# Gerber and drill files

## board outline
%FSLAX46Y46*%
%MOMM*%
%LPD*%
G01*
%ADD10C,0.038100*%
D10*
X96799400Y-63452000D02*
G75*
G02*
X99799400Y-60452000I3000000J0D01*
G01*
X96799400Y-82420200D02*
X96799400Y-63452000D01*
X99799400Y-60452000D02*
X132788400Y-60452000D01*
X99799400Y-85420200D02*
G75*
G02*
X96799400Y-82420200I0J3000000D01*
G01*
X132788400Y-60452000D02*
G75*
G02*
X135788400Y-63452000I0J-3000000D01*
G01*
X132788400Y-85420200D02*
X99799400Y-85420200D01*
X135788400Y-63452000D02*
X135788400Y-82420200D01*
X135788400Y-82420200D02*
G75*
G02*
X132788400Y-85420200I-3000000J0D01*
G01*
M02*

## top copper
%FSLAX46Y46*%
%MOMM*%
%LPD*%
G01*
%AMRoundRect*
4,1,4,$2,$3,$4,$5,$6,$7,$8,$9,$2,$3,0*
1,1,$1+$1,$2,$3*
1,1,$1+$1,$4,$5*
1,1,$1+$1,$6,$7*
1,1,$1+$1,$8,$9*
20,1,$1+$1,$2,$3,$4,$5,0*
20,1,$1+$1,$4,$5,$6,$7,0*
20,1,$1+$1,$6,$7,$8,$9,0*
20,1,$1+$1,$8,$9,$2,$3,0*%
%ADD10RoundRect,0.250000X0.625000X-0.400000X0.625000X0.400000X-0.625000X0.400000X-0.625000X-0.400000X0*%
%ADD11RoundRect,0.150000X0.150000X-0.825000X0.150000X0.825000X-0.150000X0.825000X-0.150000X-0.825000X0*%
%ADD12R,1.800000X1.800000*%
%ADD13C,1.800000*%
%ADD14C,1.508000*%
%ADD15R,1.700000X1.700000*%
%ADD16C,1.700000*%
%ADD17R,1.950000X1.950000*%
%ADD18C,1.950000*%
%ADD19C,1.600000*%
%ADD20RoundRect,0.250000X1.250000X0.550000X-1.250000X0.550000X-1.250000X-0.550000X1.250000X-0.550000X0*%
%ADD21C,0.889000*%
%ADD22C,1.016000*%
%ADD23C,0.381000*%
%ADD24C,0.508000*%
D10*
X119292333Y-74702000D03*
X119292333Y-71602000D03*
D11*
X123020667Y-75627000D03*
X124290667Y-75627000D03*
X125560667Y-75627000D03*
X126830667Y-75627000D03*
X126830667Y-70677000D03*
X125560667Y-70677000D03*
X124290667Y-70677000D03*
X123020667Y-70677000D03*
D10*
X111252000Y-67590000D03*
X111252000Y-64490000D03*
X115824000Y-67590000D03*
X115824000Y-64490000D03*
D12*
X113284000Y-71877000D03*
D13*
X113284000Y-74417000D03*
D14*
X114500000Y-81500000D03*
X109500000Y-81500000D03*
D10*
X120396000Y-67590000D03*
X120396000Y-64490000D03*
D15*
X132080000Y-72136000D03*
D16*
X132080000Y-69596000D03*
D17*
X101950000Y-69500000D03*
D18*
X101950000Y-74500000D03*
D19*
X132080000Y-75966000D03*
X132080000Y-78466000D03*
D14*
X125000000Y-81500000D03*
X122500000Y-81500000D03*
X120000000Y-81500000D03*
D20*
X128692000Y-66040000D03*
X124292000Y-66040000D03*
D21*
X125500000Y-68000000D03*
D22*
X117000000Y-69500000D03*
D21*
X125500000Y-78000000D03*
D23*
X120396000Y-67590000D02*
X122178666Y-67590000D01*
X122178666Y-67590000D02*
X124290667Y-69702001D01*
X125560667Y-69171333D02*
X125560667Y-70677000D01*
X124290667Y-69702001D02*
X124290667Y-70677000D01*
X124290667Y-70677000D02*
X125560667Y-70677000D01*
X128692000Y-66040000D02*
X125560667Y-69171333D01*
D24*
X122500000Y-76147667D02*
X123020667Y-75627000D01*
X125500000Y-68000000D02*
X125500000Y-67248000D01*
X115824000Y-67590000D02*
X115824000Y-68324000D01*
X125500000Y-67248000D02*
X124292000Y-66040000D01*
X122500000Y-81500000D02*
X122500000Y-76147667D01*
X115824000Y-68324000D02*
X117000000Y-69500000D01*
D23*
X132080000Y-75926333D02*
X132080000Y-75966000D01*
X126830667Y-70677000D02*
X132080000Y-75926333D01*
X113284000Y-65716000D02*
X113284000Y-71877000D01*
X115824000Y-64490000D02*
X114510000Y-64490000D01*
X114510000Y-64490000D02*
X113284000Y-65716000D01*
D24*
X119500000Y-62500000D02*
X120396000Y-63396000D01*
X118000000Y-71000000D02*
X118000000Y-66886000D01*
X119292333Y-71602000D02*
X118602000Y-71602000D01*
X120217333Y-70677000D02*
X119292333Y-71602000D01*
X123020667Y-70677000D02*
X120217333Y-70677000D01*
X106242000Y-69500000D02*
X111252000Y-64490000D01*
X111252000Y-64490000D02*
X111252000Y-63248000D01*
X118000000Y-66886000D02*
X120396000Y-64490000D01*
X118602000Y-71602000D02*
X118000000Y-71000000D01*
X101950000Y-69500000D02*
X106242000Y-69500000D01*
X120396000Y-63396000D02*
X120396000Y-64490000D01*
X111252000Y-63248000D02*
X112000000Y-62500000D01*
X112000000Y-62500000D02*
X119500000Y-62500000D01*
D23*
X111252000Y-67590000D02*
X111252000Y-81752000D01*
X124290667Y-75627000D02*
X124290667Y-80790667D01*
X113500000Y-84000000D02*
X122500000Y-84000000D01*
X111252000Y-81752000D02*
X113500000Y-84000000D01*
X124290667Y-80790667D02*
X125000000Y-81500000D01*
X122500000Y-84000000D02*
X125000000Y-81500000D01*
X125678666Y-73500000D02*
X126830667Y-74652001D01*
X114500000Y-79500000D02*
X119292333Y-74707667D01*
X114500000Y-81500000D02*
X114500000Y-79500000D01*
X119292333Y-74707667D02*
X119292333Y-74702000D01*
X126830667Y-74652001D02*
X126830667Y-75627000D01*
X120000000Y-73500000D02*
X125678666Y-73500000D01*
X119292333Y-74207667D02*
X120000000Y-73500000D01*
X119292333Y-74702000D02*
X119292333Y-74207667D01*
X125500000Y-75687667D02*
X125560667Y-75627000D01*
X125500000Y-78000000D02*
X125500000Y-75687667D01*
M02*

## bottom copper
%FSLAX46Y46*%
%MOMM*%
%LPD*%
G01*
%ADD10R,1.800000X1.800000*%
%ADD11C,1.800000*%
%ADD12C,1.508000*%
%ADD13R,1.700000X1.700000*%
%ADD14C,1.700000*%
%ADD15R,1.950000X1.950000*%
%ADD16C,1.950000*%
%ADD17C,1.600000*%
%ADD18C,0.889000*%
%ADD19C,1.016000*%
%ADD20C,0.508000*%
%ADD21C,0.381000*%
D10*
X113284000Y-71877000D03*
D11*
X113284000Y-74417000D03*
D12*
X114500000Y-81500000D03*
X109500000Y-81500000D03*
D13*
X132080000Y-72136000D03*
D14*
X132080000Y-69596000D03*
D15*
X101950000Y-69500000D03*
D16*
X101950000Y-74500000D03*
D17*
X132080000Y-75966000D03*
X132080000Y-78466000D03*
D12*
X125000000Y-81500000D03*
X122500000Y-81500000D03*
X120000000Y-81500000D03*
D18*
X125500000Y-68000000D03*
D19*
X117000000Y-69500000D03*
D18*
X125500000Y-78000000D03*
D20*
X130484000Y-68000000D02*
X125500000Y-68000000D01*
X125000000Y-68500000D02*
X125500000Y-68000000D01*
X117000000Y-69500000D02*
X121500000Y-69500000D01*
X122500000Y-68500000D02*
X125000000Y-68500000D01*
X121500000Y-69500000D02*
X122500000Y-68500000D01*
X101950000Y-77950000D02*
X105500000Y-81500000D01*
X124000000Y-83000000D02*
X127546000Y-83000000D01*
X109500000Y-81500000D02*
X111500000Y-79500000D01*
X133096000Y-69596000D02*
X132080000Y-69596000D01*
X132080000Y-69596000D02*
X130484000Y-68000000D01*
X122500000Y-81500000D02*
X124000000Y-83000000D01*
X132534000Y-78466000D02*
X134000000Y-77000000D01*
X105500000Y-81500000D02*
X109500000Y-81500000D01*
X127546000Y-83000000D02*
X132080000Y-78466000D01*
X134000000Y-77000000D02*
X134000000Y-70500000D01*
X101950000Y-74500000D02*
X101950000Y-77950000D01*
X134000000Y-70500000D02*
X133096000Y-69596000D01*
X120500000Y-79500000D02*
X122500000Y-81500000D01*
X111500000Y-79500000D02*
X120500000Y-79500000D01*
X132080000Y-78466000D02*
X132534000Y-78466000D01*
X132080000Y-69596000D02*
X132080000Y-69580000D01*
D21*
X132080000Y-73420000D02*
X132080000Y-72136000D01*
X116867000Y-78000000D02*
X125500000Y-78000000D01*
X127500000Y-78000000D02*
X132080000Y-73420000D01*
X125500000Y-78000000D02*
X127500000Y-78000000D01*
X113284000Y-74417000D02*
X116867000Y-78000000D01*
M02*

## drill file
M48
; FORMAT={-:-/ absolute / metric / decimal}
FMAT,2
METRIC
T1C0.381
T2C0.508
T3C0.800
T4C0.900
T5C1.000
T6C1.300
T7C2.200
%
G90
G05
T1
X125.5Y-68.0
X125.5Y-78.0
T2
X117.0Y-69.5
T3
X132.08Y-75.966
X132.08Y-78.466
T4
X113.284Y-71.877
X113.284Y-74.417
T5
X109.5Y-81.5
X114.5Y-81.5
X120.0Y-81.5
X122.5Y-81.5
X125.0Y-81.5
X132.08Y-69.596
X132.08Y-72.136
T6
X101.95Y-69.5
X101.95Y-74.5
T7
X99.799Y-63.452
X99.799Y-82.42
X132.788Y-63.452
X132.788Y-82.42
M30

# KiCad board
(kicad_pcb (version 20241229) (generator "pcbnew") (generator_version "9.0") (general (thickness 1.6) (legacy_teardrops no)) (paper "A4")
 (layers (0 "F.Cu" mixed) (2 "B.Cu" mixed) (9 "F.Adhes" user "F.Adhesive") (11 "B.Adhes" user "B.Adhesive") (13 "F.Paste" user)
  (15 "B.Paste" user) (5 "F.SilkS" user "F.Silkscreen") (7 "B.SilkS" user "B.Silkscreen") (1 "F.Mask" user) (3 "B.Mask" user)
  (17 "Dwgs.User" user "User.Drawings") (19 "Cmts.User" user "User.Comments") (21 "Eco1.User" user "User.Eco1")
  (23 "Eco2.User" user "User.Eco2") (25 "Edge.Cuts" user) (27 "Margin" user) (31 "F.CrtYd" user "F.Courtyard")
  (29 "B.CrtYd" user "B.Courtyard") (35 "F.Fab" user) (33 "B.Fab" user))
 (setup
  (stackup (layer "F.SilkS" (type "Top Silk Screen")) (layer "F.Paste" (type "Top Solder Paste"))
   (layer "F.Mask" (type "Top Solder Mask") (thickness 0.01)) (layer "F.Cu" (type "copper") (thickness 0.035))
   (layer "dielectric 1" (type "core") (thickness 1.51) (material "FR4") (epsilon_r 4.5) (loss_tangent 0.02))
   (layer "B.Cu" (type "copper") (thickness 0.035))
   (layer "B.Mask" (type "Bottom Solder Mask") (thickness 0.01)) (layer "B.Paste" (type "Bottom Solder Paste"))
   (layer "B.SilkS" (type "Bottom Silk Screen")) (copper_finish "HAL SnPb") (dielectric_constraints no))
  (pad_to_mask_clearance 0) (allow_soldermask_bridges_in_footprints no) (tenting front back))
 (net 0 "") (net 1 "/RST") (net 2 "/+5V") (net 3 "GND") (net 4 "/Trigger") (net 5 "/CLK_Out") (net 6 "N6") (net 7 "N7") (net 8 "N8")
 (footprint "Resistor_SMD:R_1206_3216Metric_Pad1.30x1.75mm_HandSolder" (layer "F.Cu") (at 119.292333 73.152 90)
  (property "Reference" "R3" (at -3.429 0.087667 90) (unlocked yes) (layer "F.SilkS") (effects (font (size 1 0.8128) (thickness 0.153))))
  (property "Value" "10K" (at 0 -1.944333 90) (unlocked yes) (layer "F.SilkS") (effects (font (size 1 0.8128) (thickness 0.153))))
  (pad "1" smd roundrect (at -1.55 0 90) (size 1.3 1.75) (layers "F.Cu" "F.Mask" "F.Paste") (roundrect_rratio 0.192308) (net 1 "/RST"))
  (pad "2" smd roundrect (at 1.55 0 90) (size 1.3 1.75) (layers "F.Cu" "F.Mask" "F.Paste") (roundrect_rratio 0.192308) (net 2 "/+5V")))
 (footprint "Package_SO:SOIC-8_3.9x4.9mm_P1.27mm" (layer "F.Cu") (at 124.925667 73.152 90)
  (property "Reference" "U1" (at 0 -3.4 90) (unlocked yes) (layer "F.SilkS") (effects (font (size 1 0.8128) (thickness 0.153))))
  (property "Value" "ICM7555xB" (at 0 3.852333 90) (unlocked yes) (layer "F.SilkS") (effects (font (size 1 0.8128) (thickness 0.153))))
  (pad "1" smd roundrect (at -2.475 -1.905 90) (size 1.95 0.6) (layers "F.Cu" "F.Mask" "F.Paste") (roundrect_rratio 0.25) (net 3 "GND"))
  (pad "2" smd roundrect (at -2.475 -0.635 90) (size 1.95 0.6) (layers "F.Cu" "F.Mask" "F.Paste") (roundrect_rratio 0.25) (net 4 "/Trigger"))
  (pad "3" smd roundrect (at -2.475 0.635 90) (size 1.95 0.6) (layers "F.Cu" "F.Mask" "F.Paste") (roundrect_rratio 0.25) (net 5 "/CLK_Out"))
  (pad "4" smd roundrect (at -2.475 1.905 90) (size 1.95 0.6) (layers "F.Cu" "F.Mask" "F.Paste") (roundrect_rratio 0.25) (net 1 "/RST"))
  (pad "5" smd roundrect (at 2.475 1.905 90) (size 1.95 0.6) (layers "F.Cu" "F.Mask" "F.Paste") (roundrect_rratio 0.25) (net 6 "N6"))
  (pad "6" smd roundrect (at 2.475 0.635 90) (size 1.95 0.6) (layers "F.Cu" "F.Mask" "F.Paste") (roundrect_rratio 0.25) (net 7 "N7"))
  (pad "7" smd roundrect (at 2.475 -0.635 90) (size 1.95 0.6) (layers "F.Cu" "F.Mask" "F.Paste") (roundrect_rratio 0.25) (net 7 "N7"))
  (pad "8" smd roundrect (at 2.475 -1.905 90) (size 1.95 0.6) (layers "F.Cu" "F.Mask" "F.Paste") (roundrect_rratio 0.25) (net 2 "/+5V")))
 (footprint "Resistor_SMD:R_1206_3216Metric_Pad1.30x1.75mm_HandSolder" (layer "F.Cu") (at 111.252 66.04 90)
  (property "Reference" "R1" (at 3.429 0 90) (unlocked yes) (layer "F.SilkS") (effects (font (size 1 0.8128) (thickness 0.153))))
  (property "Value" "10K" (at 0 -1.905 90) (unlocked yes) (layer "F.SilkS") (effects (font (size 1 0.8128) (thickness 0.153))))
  (pad "1" smd roundrect (at -1.55 0 90) (size 1.3 1.75) (layers "F.Cu" "F.Mask" "F.Paste") (roundrect_rratio 0.192308) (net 4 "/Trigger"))
  (pad "2" smd roundrect (at 1.55 0 90) (size 1.3 1.75) (layers "F.Cu" "F.Mask" "F.Paste") (roundrect_rratio 0.192308) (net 2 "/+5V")))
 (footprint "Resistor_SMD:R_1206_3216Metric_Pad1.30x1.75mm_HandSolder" (layer "F.Cu") (at 115.824 66.04 90)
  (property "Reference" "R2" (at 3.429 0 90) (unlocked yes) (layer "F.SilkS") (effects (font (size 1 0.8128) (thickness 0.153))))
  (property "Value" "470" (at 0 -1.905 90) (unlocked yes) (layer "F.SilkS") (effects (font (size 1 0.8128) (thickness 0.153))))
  (pad "1" smd roundrect (at -1.55 0 90) (size 1.3 1.75) (layers "F.Cu" "F.Mask" "F.Paste") (roundrect_rratio 0.192308) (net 3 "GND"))
  (pad "2" smd roundrect (at 1.55 0 90) (size 1.3 1.75) (layers "F.Cu" "F.Mask" "F.Paste") (roundrect_rratio 0.192308) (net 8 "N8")))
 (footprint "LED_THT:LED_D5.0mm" (layer "F.Cu") (at 113.284 71.877 -90)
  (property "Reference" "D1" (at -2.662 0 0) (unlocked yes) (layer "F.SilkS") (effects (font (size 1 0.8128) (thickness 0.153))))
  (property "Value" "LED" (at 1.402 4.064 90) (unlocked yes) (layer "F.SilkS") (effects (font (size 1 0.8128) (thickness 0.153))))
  (pad "1" thru_hole rect (at 0 0 270) (size 1.8 1.8) (drill 0.9) (layers "*.Cu" "*.Mask") (remove_unused_layers no) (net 8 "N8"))
  (pad "2" thru_hole circle (at 2.54 0 270) (size 1.8 1.8) (drill 0.9) (layers "*.Cu" "*.Mask") (remove_unused_layers no) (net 5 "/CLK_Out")))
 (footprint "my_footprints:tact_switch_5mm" (layer "F.Cu") (at 112 81.5 180)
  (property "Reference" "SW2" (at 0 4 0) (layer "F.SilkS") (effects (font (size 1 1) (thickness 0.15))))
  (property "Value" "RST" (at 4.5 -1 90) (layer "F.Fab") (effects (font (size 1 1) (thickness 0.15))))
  (pad "1" thru_hole circle (at -2.5 0 180) (size 1.508 1.508) (drill 1) (layers "*.Cu" "*.Mask") (remove_unused_layers no) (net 1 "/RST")
   (solder_mask_margin 0.102))
  (pad "2" thru_hole circle (at 2.5 0 180) (size 1.508 1.508) (drill 1) (layers "*.Cu" "*.Mask") (remove_unused_layers no) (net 3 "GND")
   (solder_mask_margin 0.102)))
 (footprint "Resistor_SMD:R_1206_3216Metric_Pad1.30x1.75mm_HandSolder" (layer "F.Cu") (at 120.396 66.04 90)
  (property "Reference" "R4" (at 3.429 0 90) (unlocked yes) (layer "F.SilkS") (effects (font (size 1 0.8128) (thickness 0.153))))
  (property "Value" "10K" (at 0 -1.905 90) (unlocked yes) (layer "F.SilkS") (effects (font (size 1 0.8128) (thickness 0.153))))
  (pad "1" smd roundrect (at -1.55 0 90) (size 1.3 1.75) (layers "F.Cu" "F.Mask" "F.Paste") (roundrect_rratio 0.192308) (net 7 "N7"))
  (pad "2" smd roundrect (at 1.55 0 90) (size 1.3 1.75) (layers "F.Cu" "F.Mask" "F.Paste") (roundrect_rratio 0.192308) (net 2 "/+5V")))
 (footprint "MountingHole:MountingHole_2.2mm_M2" (layer "F.Cu") (at 99.7994 63.452)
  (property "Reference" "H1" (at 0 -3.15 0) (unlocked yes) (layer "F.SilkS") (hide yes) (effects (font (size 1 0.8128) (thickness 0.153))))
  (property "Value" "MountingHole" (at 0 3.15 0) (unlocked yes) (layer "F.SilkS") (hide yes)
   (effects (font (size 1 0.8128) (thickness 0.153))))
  (pad "" np_thru_hole circle (at 0 0) (size 2.2 2.2) (drill 2.2) (layers "*.Cu" "*.Mask")))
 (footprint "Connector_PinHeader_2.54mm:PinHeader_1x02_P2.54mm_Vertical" (layer "F.Cu") (at 132.08 72.136 180)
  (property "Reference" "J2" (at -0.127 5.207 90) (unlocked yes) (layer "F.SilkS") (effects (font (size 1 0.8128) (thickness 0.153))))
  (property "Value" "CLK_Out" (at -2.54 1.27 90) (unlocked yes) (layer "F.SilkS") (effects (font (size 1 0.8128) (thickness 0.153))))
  (pad "1" thru_hole rect (at 0 0 180) (size 1.7 1.7) (drill 1) (layers "*.Cu" "*.Mask") (remove_unused_layers no) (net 5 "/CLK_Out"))
  (pad "2" thru_hole circle (at 0 2.54 180) (size 1.7 1.7) (drill 1) (layers "*.Cu" "*.Mask") (remove_unused_layers no) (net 3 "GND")))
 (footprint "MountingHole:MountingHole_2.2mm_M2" (layer "F.Cu") (at 132.7884 82.4202)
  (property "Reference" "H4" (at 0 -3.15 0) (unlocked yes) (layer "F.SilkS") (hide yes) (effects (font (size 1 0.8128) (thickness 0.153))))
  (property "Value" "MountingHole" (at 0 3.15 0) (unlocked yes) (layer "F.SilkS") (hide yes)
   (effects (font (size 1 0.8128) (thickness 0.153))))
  (pad "" np_thru_hole circle (at 0 0) (size 2.2 2.2) (drill 2.2) (layers "*.Cu" "*.Mask")))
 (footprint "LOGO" (layer "F.Cu") (at 105.5 63.5)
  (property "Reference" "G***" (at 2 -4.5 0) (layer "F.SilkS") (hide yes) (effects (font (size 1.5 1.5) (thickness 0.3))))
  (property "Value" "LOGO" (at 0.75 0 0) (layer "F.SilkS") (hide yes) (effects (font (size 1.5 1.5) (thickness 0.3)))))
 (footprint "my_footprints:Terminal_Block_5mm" (layer "F.Cu") (at 101.95 72 -90)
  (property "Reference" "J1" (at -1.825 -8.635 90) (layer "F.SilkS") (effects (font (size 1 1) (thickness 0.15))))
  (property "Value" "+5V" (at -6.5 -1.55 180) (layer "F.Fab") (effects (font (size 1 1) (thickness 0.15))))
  (pad "1" thru_hole rect (at -2.5 0 270) (size 1.95 1.95) (drill 1.3) (layers "*.Cu" "*.Mask") (remove_unused_layers no) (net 2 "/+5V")
   (solder_mask_margin 0.102))
  (pad "2" thru_hole circle (at 2.5 0 270) (size 1.95 1.95) (drill 1.3) (layers "*.Cu" "*.Mask") (remove_unused_layers no) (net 3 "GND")
   (solder_mask_margin 0.102)))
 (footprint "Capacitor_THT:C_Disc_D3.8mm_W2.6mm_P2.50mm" (layer "F.Cu") (at 132.08 75.966 -90)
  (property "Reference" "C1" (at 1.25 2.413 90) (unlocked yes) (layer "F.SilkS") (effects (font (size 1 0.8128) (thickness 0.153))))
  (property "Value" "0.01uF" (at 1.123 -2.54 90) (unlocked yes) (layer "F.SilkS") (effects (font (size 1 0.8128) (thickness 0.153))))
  (pad "1" thru_hole circle (at 0 0 270) (size 1.6 1.6) (drill 0.8) (layers "*.Cu" "*.Mask") (remove_unused_layers no) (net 6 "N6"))
  (pad "2" thru_hole circle (at 2.5 0 270) (size 1.6 1.6) (drill 0.8) (layers "*.Cu" "*.Mask") (remove_unused_layers no) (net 3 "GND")))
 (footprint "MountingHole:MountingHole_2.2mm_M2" (layer "F.Cu") (at 132.7884 63.452)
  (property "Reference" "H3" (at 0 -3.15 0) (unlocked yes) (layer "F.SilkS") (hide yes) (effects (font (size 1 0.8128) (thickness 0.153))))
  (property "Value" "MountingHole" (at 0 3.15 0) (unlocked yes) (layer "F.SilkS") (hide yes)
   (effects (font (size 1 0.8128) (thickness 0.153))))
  (pad "" np_thru_hole circle (at 0 0) (size 2.2 2.2) (drill 2.2) (layers "*.Cu" "*.Mask")))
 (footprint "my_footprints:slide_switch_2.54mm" (layer "F.Cu") (at 122.5 81.5 180)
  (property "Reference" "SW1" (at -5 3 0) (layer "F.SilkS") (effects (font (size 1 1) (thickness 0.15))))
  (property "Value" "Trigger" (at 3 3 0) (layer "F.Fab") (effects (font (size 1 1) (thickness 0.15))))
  (pad "1" thru_hole circle (at -2.5 0 180) (size 1.508 1.508) (drill 1) (layers "*.Cu" "*.Mask") (remove_unused_layers no)
   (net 4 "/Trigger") (solder_mask_margin 0.102))
  (pad "2" thru_hole circle (at 0 0 180) (size 1.508 1.508) (drill 1) (layers "*.Cu" "*.Mask") (remove_unused_layers no) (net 3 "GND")
   (solder_mask_margin 0.102))
  (pad "3" thru_hole circle (at 2.5 0 180) (size 1.508 1.508) (drill 1) (layers "*.Cu" "*.Mask") (remove_unused_layers no)
   (solder_mask_margin 0.102)))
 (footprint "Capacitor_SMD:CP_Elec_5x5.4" (layer "F.Cu") (at 126.492 66.04 180)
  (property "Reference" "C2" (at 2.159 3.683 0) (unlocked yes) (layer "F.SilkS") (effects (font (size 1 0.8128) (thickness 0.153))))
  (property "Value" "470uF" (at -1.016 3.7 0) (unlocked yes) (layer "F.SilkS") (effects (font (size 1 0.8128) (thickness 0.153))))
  (pad "1" smd roundrect (at -2.2 0 180) (size 3 1.6) (layers "F.Cu" "F.Mask" "F.Paste") (roundrect_rratio 0.15625) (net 7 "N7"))
  (pad "2" smd roundrect (at 2.2 0 180) (size 3 1.6) (layers "F.Cu" "F.Mask" "F.Paste") (roundrect_rratio 0.15625) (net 3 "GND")))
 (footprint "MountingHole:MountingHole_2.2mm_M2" (layer "F.Cu") (at 99.7994 82.4202)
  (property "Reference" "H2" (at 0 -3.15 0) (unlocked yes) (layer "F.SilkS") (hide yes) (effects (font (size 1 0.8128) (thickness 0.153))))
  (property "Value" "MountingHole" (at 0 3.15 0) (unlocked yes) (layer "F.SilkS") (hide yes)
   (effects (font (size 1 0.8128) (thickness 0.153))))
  (pad "" np_thru_hole circle (at 0 0) (size 2.2 2.2) (drill 2.2) (layers "*.Cu" "*.Mask")))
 (gr_arc (start 96.7994 63.452) (mid 97.67808 61.33068) (end 99.7994 60.452) (stroke (width 0.0381) (type default)) (layer "Edge.Cuts"))
 (gr_line (start 96.7994 82.4202) (end 96.7994 63.452) (stroke (width 0.0381) (type default)) (layer "Edge.Cuts"))
 (gr_line (start 99.7994 60.452) (end 132.7884 60.452) (stroke (width 0.0381) (type default)) (layer "Edge.Cuts"))
 (gr_arc (start 99.7994 85.4202) (mid 97.67808 84.54152) (end 96.7994 82.4202) (stroke (width 0.0381) (type default)) (layer "Edge.Cuts"))
 (gr_arc (start 132.7884 60.452) (mid 134.90972 61.33068) (end 135.7884 63.452) (stroke (width 0.0381) (type default)) (layer "Edge.Cuts"))
 (gr_line (start 132.7884 85.4202) (end 99.7994 85.4202) (stroke (width 0.0381) (type default)) (layer "Edge.Cuts"))
 (gr_line (start 135.7884 63.452) (end 135.7884 82.4202) (stroke (width 0.0381) (type default)) (layer "Edge.Cuts"))
 (gr_arc (start 135.7884 82.4202) (mid 134.90972 84.54152) (end 132.7884 85.4202) (stroke (width 0.0381) (type default)) (layer "Edge.Cuts"))
 (segment (start 120.396 67.59) (end 122.178666 67.59) (width 0.381) (layer "F.Cu") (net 7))
 (segment (start 122.178666 67.59) (end 124.290667 69.702001) (width 0.381) (layer "F.Cu") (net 7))
 (segment (start 125.560667 69.171333) (end 125.560667 70.677) (width 0.381) (layer "F.Cu") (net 7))
 (segment (start 124.290667 69.702001) (end 124.290667 70.677) (width 0.381) (layer "F.Cu") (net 7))
 (segment (start 124.290667 70.677) (end 125.560667 70.677) (width 0.381) (layer "F.Cu") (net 7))
 (segment (start 128.692 66.04) (end 125.560667 69.171333) (width 0.381) (layer "F.Cu") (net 7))
 (segment (start 122.5 76.147667) (end 123.020667 75.627) (width 0.508) (layer "F.Cu") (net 3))
 (segment (start 125.5 68) (end 125.5 67.248) (width 0.508) (layer "F.Cu") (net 3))
 (segment (start 115.824 67.59) (end 115.824 68.324) (width 0.508) (layer "F.Cu") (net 3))
 (segment (start 125.5 67.248) (end 124.292 66.04) (width 0.508) (layer "F.Cu") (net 3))
 (segment (start 122.5 81.5) (end 122.5 76.147667) (width 0.508) (layer "F.Cu") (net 3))
 (segment (start 115.824 68.324) (end 117 69.5) (width 0.508) (layer "F.Cu") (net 3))
 (via (at 125.5 68) (size 0.889) (drill 0.381) (layers "F.Cu" "B.Cu") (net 3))
 (via (at 117 69.5) (size 1.016) (drill 0.508) (layers "F.Cu" "B.Cu") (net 3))
 (segment (start 130.484 68) (end 125.5 68) (width 0.508) (layer "B.Cu") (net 3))
 (segment (start 125 68.5) (end 125.5 68) (width 0.508) (layer "B.Cu") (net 3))
 (segment (start 117 69.5) (end 121.5 69.5) (width 0.508) (layer "B.Cu") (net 3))
 (segment (start 122.5 68.5) (end 125 68.5) (width 0.508) (layer "B.Cu") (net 3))
 (segment (start 121.5 69.5) (end 122.5 68.5) (width 0.508) (layer "B.Cu") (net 3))
 (segment (start 101.95 77.95) (end 105.5 81.5) (width 0.508) (layer "B.Cu") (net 3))
 (segment (start 124 83) (end 127.546 83) (width 0.508) (layer "B.Cu") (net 3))
 (segment (start 109.5 81.5) (end 111.5 79.5) (width 0.508) (layer "B.Cu") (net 3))
 (segment (start 133.096 69.596) (end 132.08 69.596) (width 0.508) (layer "B.Cu") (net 3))
 (segment (start 132.08 69.596) (end 130.484 68) (width 0.508) (layer "B.Cu") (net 3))
 (segment (start 122.5 81.5) (end 124 83) (width 0.508) (layer "B.Cu") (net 3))
 (segment (start 132.534 78.466) (end 134 77) (width 0.508) (layer "B.Cu") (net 3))
 (segment (start 105.5 81.5) (end 109.5 81.5) (width 0.508) (layer "B.Cu") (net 3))
 (segment (start 127.546 83) (end 132.08 78.466) (width 0.508) (layer "B.Cu") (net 3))
 (segment (start 134 77) (end 134 70.5) (width 0.508) (layer "B.Cu") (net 3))
 (segment (start 101.95 74.5) (end 101.95 77.95) (width 0.508) (layer "B.Cu") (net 3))
 (segment (start 134 70.5) (end 133.096 69.596) (width 0.508) (layer "B.Cu") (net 3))
 (segment (start 120.5 79.5) (end 122.5 81.5) (width 0.508) (layer "B.Cu") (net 3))
 (segment (start 111.5 79.5) (end 120.5 79.5) (width 0.508) (layer "B.Cu") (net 3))
 (segment (start 132.08 78.466) (end 132.534 78.466) (width 0.508) (layer "B.Cu") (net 3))
 (segment (start 132.08 69.596) (end 132.08 69.58) (width 0.508) (layer "B.Cu") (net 3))
 (segment (start 132.08 75.926333) (end 132.08 75.966) (width 0.381) (layer "F.Cu") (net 6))
 (segment (start 126.830667 70.677) (end 132.08 75.926333) (width 0.381) (layer "F.Cu") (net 6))
 (segment (start 113.284 65.716) (end 113.284 71.877) (width 0.381) (layer "F.Cu") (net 8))
 (segment (start 115.824 64.49) (end 114.51 64.49) (width 0.381) (layer "F.Cu") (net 8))
 (segment (start 114.51 64.49) (end 113.284 65.716) (width 0.381) (layer "F.Cu") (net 8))
 (segment (start 119.5 62.5) (end 120.396 63.396) (width 0.508) (layer "F.Cu") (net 2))
 (segment (start 118 71) (end 118 66.886) (width 0.508) (layer "F.Cu") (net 2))
 (segment (start 119.292333 71.602) (end 118.602 71.602) (width 0.508) (layer "F.Cu") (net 2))
 (segment (start 120.217333 70.677) (end 119.292333 71.602) (width 0.508) (layer "F.Cu") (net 2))
 (segment (start 123.020667 70.677) (end 120.217333 70.677) (width 0.508) (layer "F.Cu") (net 2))
 (segment (start 106.242 69.5) (end 111.252 64.49) (width 0.508) (layer "F.Cu") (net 2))
 (segment (start 111.252 64.49) (end 111.252 63.248) (width 0.508) (layer "F.Cu") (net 2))
 (segment (start 118 66.886) (end 120.396 64.49) (width 0.508) (layer "F.Cu") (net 2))
 (segment (start 118.602 71.602) (end 118 71) (width 0.508) (layer "F.Cu") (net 2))
 (segment (start 101.95 69.5) (end 106.242 69.5) (width 0.508) (layer "F.Cu") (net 2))
 (segment (start 120.396 63.396) (end 120.396 64.49) (width 0.508) (layer "F.Cu") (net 2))
 (segment (start 111.252 63.248) (end 112 62.5) (width 0.508) (layer "F.Cu") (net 2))
 (segment (start 112 62.5) (end 119.5 62.5) (width 0.508) (layer "F.Cu") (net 2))
 (segment (start 111.252 67.59) (end 111.252 81.752) (width 0.381) (layer "F.Cu") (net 4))
 (segment (start 124.290667 75.627) (end 124.290667 80.790667) (width 0.381) (layer "F.Cu") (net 4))
 (segment (start 113.5 84) (end 122.5 84) (width 0.381) (layer "F.Cu") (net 4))
 (segment (start 111.252 81.752) (end 113.5 84) (width 0.381) (layer "F.Cu") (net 4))
 (segment (start 124.290667 80.790667) (end 125 81.5) (width 0.381) (layer "F.Cu") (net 4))
 (segment (start 122.5 84) (end 125 81.5) (width 0.381) (layer "F.Cu") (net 4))
 (segment (start 125.678666 73.5) (end 126.830667 74.652001) (width 0.381) (layer "F.Cu") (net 1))
 (segment (start 114.5 79.5) (end 119.292333 74.707667) (width 0.381) (layer "F.Cu") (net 1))
 (segment (start 114.5 81.5) (end 114.5 79.5) (width 0.381) (layer "F.Cu") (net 1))
 (segment (start 119.292333 74.707667) (end 119.292333 74.702) (width 0.381) (layer "F.Cu") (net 1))
 (segment (start 126.830667 74.652001) (end 126.830667 75.627) (width 0.381) (layer "F.Cu") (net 1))
 (segment (start 120 73.5) (end 125.678666 73.5) (width 0.381) (layer "F.Cu") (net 1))
 (segment (start 119.292333 74.207667) (end 120 73.5) (width 0.381) (layer "F.Cu") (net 1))
 (segment (start 119.292333 74.702) (end 119.292333 74.207667) (width 0.381) (layer "F.Cu") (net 1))
 (segment (start 125.5 75.687667) (end 125.560667 75.627) (width 0.381) (layer "F.Cu") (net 5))
 (segment (start 125.5 78) (end 125.5 75.687667) (width 0.381) (layer "F.Cu") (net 5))
 (via (at 125.5 78) (size 0.889) (drill 0.381) (layers "F.Cu" "B.Cu") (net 5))
 (segment (start 132.08 73.42) (end 132.08 72.136) (width 0.381) (layer "B.Cu") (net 5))
 (segment (start 116.867 78) (end 125.5 78) (width 0.381) (layer "B.Cu") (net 5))
 (segment (start 127.5 78) (end 132.08 73.42) (width 0.381) (layer "B.Cu") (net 5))
 (segment (start 125.5 78) (end 127.5 78) (width 0.381) (layer "B.Cu") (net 5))
 (segment (start 113.284 74.417) (end 116.867 78) (width 0.381) (layer "B.Cu") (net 5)))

